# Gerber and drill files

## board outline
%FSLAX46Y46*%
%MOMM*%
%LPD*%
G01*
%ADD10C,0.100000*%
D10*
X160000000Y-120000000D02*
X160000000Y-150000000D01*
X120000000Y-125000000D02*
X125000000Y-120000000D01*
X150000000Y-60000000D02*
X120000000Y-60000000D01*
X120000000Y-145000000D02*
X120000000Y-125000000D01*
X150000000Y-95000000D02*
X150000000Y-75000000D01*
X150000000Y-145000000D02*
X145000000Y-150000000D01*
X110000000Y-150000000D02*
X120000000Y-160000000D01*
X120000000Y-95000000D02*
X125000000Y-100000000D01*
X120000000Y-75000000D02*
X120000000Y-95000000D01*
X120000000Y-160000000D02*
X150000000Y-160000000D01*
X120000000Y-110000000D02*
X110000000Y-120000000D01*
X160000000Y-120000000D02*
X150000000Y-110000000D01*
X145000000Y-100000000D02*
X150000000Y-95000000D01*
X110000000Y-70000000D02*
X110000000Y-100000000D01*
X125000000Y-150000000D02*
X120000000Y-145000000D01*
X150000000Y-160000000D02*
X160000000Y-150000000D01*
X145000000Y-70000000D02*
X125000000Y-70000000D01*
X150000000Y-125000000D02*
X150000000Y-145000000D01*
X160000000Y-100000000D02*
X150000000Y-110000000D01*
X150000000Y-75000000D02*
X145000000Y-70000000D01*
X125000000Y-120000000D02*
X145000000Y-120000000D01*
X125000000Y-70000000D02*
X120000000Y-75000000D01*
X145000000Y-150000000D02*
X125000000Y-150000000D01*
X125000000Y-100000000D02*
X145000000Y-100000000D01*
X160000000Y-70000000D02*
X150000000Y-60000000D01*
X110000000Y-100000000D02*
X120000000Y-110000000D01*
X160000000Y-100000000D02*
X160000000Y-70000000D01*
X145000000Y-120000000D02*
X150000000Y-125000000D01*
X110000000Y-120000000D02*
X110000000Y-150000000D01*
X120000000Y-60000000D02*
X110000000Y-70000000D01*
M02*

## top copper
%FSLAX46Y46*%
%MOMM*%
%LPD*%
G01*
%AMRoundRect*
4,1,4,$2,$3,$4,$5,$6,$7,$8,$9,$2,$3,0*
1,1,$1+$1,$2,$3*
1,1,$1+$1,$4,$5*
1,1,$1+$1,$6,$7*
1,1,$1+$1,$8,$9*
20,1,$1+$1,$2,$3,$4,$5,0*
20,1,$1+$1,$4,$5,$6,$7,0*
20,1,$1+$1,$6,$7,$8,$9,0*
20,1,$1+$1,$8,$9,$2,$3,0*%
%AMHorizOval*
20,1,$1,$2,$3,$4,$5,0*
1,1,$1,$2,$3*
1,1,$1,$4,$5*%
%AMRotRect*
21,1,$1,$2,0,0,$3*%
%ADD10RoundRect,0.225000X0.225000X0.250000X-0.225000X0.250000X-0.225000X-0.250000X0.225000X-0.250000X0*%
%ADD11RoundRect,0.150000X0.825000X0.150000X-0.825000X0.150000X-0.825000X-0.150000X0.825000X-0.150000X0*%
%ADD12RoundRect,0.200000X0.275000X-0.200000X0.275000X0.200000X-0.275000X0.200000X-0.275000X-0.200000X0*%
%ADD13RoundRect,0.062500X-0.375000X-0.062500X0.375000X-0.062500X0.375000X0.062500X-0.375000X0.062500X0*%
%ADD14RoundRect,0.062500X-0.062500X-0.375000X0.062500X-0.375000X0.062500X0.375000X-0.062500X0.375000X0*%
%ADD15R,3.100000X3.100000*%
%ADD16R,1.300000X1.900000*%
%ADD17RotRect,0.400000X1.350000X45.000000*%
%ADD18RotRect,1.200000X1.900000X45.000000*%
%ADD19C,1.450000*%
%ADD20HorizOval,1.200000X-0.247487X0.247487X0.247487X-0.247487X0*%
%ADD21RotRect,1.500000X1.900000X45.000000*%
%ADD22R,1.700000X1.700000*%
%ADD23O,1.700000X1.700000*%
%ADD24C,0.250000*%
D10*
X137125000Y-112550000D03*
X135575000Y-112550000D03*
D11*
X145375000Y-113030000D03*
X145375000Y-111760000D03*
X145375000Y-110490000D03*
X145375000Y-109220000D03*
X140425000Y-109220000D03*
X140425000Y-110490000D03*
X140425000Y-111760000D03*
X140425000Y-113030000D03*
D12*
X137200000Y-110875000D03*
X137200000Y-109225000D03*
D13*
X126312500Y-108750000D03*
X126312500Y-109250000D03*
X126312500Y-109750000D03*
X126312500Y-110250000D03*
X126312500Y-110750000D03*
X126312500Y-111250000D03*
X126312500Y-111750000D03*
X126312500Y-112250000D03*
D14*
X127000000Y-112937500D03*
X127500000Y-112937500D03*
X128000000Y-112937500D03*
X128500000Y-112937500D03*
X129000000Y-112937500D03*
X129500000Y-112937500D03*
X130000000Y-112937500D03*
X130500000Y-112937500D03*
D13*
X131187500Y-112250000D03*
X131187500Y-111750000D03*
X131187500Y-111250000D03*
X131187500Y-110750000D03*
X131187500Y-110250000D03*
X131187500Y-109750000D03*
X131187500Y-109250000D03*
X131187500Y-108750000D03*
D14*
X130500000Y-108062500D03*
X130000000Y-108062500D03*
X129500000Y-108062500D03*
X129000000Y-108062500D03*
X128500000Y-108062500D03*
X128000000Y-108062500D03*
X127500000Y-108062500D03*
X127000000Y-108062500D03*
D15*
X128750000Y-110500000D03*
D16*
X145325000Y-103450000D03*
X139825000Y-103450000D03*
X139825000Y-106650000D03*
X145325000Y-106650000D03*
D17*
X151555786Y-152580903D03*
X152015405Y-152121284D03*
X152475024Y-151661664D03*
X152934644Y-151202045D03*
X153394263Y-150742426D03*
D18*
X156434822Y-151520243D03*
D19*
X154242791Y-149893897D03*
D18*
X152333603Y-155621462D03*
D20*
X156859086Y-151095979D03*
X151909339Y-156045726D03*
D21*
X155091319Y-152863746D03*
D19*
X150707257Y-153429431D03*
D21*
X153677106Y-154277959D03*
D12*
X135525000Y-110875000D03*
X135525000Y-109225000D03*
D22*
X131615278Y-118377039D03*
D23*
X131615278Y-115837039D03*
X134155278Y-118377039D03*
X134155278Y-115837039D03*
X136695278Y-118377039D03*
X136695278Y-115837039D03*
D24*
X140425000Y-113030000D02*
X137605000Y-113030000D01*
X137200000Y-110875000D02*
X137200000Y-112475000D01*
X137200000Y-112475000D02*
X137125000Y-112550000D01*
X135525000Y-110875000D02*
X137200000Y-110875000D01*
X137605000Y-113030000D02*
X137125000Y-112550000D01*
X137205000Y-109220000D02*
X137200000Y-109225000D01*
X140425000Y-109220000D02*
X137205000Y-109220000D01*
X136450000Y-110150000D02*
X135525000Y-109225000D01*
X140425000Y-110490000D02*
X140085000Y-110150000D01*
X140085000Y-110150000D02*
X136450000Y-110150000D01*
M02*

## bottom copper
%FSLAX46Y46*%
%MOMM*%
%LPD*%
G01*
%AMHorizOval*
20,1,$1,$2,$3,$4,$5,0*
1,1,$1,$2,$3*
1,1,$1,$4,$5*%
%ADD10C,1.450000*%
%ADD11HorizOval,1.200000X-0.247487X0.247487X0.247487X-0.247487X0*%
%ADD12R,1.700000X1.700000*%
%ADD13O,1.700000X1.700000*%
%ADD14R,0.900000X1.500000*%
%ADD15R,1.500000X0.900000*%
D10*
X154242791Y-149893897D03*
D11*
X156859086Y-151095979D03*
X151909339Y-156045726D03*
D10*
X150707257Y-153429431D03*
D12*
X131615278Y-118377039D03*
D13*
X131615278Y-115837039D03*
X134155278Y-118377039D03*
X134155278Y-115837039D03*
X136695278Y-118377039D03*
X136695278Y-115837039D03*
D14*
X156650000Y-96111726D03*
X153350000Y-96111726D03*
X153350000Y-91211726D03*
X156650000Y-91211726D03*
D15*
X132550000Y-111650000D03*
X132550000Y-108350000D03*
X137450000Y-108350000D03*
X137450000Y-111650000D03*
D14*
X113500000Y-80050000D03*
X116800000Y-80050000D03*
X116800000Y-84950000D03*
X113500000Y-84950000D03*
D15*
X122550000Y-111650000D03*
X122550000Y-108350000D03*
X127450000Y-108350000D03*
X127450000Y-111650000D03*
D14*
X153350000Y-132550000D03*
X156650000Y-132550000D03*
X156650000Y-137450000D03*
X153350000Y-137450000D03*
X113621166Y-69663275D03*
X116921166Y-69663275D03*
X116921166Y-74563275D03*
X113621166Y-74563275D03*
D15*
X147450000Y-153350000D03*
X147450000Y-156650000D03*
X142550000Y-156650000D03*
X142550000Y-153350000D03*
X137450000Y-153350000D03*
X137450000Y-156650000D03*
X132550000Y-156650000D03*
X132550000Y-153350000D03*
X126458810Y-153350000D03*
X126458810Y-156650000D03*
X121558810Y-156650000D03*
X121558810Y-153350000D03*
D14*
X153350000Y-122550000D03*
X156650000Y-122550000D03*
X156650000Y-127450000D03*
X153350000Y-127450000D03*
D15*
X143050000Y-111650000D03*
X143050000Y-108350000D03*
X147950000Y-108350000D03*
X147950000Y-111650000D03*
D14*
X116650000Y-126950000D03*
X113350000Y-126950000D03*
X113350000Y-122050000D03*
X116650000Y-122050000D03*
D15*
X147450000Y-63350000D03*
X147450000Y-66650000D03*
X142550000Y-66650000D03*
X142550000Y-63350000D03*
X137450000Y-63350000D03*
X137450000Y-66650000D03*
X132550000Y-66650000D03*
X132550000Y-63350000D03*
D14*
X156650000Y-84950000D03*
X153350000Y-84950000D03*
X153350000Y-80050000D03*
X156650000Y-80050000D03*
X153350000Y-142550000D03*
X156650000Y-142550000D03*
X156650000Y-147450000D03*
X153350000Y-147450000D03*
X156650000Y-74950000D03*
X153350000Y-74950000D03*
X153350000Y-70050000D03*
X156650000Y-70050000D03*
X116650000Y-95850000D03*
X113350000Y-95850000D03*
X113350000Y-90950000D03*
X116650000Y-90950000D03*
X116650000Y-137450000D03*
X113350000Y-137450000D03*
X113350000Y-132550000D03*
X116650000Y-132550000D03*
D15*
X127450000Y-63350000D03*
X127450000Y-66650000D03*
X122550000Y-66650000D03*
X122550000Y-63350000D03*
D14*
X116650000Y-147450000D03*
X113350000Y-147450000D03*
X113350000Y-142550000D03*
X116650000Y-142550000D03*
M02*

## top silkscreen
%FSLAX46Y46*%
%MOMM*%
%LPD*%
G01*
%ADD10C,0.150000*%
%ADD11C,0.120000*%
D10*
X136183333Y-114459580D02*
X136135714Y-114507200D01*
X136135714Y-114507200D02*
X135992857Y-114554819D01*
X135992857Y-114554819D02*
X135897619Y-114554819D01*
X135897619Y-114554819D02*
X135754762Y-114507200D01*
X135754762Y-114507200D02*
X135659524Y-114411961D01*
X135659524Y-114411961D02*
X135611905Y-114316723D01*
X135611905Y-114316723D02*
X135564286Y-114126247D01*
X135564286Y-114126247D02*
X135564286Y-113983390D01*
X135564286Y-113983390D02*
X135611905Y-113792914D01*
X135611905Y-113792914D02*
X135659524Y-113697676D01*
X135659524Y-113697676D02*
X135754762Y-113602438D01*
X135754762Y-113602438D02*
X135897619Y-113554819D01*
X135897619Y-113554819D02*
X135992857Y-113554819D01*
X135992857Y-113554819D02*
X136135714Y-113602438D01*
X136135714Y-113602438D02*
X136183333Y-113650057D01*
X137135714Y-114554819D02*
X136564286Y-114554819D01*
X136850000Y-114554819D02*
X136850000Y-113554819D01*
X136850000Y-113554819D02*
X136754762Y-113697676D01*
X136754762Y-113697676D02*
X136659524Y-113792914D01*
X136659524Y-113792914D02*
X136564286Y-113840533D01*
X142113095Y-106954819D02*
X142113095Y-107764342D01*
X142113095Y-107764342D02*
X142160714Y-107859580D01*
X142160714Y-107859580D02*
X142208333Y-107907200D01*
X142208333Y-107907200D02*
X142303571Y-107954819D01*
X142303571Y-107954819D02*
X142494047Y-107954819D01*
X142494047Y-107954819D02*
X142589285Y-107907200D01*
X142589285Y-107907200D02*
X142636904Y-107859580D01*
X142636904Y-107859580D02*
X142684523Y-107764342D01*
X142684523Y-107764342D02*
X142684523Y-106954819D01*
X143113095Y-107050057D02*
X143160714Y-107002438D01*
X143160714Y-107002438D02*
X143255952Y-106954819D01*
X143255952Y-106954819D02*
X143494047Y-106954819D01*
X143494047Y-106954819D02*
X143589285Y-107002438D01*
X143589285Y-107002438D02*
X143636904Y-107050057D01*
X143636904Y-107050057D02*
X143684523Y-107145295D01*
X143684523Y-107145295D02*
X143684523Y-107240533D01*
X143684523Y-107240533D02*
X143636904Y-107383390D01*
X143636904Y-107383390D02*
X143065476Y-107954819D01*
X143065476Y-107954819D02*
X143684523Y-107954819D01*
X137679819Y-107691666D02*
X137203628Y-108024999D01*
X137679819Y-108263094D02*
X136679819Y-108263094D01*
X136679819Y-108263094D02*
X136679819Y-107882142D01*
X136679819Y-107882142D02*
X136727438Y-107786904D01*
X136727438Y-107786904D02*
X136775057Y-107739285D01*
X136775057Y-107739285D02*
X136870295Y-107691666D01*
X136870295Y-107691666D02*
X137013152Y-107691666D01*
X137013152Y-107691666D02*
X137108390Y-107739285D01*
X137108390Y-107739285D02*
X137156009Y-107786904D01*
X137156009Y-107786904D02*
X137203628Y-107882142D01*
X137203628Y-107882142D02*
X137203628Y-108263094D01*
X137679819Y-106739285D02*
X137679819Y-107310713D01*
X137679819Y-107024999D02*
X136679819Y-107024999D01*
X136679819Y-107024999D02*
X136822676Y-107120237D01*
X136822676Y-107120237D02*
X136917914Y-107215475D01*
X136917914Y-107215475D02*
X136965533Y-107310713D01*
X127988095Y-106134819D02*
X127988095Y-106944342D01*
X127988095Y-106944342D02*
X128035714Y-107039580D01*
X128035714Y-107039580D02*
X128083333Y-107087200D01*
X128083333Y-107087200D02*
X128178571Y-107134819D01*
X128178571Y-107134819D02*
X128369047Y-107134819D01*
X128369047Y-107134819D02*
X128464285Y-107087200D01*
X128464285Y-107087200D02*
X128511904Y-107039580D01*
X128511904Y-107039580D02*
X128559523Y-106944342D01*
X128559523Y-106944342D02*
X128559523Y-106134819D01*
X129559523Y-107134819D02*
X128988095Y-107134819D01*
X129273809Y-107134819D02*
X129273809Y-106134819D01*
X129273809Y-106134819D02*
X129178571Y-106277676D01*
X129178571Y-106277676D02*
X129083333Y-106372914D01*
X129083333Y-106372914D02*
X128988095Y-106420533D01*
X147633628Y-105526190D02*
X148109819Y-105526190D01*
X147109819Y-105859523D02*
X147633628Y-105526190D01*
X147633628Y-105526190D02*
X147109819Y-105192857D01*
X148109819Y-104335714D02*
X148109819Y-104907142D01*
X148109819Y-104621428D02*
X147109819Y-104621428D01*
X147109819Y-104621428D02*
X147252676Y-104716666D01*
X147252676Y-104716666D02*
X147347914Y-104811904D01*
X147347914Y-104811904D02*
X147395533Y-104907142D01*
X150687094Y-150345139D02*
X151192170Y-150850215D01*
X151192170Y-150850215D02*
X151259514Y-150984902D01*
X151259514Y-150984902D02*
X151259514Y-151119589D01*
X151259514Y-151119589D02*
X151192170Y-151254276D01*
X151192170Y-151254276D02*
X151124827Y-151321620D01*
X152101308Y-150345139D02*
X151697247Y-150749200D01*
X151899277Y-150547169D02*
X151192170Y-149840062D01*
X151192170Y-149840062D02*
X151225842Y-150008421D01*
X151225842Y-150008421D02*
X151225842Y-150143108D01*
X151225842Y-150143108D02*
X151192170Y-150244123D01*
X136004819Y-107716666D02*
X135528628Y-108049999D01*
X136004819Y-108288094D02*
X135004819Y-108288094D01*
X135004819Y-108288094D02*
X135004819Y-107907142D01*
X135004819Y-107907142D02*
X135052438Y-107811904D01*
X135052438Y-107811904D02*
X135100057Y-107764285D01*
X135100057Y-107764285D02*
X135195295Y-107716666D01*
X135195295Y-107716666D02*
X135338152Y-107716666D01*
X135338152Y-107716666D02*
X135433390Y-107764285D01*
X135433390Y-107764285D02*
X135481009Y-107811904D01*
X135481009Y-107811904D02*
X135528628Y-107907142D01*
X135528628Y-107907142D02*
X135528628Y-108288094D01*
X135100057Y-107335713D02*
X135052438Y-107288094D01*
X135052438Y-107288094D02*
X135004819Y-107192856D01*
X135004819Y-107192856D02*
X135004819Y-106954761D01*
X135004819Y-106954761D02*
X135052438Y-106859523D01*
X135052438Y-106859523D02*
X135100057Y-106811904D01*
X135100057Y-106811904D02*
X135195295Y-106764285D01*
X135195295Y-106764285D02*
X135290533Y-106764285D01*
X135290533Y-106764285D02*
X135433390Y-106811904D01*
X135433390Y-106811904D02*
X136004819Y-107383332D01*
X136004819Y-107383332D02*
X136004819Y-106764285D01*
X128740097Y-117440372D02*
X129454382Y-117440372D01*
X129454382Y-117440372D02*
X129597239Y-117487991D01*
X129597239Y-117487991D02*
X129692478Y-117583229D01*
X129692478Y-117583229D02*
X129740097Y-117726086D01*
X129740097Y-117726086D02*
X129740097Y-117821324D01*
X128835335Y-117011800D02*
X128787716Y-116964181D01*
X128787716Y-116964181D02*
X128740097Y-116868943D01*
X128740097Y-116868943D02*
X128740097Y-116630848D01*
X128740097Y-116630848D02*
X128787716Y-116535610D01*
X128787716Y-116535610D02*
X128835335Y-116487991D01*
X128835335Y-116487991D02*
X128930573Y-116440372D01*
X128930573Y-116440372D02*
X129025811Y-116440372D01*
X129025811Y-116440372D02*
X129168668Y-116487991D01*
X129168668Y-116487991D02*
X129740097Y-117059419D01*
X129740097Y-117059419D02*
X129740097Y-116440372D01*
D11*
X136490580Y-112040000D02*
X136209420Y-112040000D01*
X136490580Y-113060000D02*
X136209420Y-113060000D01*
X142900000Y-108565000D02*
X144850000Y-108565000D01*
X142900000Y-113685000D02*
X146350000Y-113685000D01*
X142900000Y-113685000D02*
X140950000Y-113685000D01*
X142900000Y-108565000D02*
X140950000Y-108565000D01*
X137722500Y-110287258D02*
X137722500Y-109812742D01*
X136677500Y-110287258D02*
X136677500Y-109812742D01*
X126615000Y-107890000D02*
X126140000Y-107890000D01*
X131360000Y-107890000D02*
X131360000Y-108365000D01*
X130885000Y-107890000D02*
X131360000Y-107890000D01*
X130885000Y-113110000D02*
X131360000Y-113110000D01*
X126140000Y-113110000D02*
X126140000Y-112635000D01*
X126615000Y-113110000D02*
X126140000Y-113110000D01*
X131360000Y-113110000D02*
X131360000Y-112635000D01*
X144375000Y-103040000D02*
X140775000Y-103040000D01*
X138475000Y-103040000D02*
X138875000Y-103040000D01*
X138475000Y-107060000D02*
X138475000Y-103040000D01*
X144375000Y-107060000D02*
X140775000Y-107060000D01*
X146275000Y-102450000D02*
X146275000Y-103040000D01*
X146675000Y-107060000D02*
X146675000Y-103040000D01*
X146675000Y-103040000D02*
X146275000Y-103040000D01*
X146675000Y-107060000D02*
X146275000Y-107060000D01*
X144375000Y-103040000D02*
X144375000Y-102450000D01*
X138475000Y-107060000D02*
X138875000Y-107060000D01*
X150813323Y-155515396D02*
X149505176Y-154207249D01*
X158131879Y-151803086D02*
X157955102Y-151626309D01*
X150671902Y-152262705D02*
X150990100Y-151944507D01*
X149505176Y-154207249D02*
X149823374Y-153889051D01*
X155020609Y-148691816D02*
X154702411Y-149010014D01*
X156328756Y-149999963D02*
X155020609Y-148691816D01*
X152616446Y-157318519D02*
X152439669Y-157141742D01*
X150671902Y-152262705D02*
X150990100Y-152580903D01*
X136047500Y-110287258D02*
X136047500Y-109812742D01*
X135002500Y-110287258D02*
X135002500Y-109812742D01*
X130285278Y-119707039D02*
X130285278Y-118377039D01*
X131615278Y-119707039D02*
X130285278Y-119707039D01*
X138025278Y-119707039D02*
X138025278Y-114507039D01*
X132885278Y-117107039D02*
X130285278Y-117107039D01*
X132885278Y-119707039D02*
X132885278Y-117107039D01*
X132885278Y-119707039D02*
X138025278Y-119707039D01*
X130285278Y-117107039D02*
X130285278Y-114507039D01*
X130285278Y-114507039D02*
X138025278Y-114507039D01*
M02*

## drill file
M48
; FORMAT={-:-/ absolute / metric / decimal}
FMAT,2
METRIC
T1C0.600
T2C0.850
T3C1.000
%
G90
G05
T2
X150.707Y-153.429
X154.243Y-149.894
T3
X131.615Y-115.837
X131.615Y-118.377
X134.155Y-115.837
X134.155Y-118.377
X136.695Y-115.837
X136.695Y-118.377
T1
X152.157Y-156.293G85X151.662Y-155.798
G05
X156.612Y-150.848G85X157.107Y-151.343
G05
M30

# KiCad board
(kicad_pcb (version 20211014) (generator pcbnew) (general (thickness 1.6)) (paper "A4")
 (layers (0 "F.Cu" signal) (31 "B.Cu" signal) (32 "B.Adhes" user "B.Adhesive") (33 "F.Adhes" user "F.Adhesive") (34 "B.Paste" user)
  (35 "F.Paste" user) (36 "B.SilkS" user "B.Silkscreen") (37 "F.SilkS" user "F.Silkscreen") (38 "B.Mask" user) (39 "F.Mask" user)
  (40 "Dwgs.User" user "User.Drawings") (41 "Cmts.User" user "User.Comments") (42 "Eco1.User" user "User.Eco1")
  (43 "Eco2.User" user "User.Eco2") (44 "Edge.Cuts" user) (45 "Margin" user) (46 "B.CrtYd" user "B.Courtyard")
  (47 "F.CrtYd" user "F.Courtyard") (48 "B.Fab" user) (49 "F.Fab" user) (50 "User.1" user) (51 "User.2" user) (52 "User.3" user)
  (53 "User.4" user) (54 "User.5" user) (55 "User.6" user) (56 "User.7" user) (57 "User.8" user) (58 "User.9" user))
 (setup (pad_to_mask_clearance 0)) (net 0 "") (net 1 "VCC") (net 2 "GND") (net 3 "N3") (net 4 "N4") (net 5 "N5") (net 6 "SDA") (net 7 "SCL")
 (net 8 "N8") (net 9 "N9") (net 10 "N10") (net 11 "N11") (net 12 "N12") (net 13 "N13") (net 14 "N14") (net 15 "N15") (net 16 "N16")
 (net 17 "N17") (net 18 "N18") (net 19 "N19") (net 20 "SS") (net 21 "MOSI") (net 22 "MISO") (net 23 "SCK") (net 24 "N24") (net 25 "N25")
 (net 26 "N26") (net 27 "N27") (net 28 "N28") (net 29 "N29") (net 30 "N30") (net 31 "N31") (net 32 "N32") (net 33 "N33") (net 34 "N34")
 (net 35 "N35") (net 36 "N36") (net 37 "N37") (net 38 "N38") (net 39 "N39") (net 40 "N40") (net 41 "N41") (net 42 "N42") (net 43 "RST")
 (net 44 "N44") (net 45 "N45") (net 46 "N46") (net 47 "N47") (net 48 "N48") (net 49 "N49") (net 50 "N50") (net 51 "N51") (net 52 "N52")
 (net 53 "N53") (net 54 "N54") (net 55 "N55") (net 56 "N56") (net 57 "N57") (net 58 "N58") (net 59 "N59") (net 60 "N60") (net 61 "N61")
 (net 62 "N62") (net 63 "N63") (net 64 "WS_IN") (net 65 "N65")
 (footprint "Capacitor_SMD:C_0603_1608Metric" (layer "F.Cu") (at 136.35 112.55 180)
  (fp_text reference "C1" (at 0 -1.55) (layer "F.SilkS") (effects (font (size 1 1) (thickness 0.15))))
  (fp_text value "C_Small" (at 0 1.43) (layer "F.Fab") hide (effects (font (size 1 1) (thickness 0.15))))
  (fp_line (start -0.14058 0.51) (end 0.14058 0.51) (layer "F.SilkS") (width 0.12))
  (fp_line (start -0.14058 -0.51) (end 0.14058 -0.51) (layer "F.SilkS") (width 0.12))
  (pad "1" smd roundrect (at -0.775 0 180) (size 0.9 0.95) (layers "F.Cu" "F.Paste" "F.Mask") (roundrect_rratio 0.25) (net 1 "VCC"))
  (pad "2" smd roundrect (at 0.775 0 180) (size 0.9 0.95) (layers "F.Cu" "F.Paste" "F.Mask") (roundrect_rratio 0.25) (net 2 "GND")))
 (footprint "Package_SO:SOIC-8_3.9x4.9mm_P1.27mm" (layer "F.Cu") (at 142.9 111.125 180)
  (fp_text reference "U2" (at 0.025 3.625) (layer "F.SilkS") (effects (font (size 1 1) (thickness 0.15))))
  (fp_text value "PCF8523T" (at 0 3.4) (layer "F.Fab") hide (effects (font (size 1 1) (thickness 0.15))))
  (fp_line (start 0 2.56) (end -1.95 2.56) (layer "F.SilkS") (width 0.12))
  (fp_line (start 0 -2.56) (end -3.45 -2.56) (layer "F.SilkS") (width 0.12))
  (fp_line (start 0 -2.56) (end 1.95 -2.56) (layer "F.SilkS") (width 0.12))
  (fp_line (start 0 2.56) (end 1.95 2.56) (layer "F.SilkS") (width 0.12))
  (pad "1" smd roundrect (at -2.475 -1.905 180) (size 1.95 0.6) (layers "F.Cu" "F.Paste" "F.Mask") (roundrect_rratio 0.25) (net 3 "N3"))
  (pad "2" smd roundrect (at -2.475 -0.635 180) (size 1.95 0.6) (layers "F.Cu" "F.Paste" "F.Mask") (roundrect_rratio 0.25) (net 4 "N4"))
  (pad "3" smd roundrect (at -2.475 0.635 180) (size 1.95 0.6) (layers "F.Cu" "F.Paste" "F.Mask") (roundrect_rratio 0.25) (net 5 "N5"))
  (pad "4" smd roundrect (at -2.475 1.905 180) (size 1.95 0.6) (layers "F.Cu" "F.Paste" "F.Mask") (roundrect_rratio 0.25) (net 2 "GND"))
  (pad "5" smd roundrect (at 2.475 1.905 180) (size 1.95 0.6) (layers "F.Cu" "F.Paste" "F.Mask") (roundrect_rratio 0.25) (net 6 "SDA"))
  (pad "6" smd roundrect (at 2.475 0.635 180) (size 1.95 0.6) (layers "F.Cu" "F.Paste" "F.Mask") (roundrect_rratio 0.25) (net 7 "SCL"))
  (pad "7" smd roundrect (at 2.475 -0.635 180) (size 1.95 0.6) (layers "F.Cu" "F.Paste" "F.Mask") (roundrect_rratio 0.25) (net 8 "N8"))
  (pad "8" smd roundrect (at 2.475 -1.905 180) (size 1.95 0.6) (layers "F.Cu" "F.Paste" "F.Mask") (roundrect_rratio 0.25) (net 1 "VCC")))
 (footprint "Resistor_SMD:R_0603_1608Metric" (layer "F.Cu") (at 137.2 110.05 90)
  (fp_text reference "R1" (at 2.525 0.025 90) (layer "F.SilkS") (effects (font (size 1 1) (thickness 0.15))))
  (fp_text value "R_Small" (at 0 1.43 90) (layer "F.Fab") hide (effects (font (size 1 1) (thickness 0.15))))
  (fp_line (start -0.237258 0.5225) (end 0.237258 0.5225) (layer "F.SilkS") (width 0.12))
  (fp_line (start -0.237258 -0.5225) (end 0.237258 -0.5225) (layer "F.SilkS") (width 0.12))
  (pad "1" smd roundrect (at -0.825 0 90) (size 0.8 0.95) (layers "F.Cu" "F.Paste" "F.Mask") (roundrect_rratio 0.25) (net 1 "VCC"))
  (pad "2" smd roundrect (at 0.825 0 90) (size 0.8 0.95) (layers "F.Cu" "F.Paste" "F.Mask") (roundrect_rratio 0.25) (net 6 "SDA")))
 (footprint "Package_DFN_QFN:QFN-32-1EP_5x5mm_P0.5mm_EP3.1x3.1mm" (layer "F.Cu") (at 128.75 110.5)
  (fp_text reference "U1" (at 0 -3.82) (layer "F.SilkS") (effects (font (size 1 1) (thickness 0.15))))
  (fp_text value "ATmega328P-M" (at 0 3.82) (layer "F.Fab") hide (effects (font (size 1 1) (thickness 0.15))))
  (fp_line (start -2.135 -2.61) (end -2.61 -2.61) (layer "F.SilkS") (width 0.12))
  (fp_line (start 2.61 -2.61) (end 2.61 -2.135) (layer "F.SilkS") (width 0.12))
  (fp_line (start 2.135 -2.61) (end 2.61 -2.61) (layer "F.SilkS") (width 0.12))
  (fp_line (start 2.135 2.61) (end 2.61 2.61) (layer "F.SilkS") (width 0.12))
  (fp_line (start -2.61 2.61) (end -2.61 2.135) (layer "F.SilkS") (width 0.12))
  (fp_line (start -2.135 2.61) (end -2.61 2.61) (layer "F.SilkS") (width 0.12))
  (fp_line (start 2.61 2.61) (end 2.61 2.135) (layer "F.SilkS") (width 0.12))
  (pad "" smd roundrect (at 1.03 -1.03) (size 0.83 0.83) (layers "F.Paste") (roundrect_rratio 0.25))
  (pad "" smd roundrect (at -1.03 -1.03) (size 0.83 0.83) (layers "F.Paste") (roundrect_rratio 0.25))
  (pad "" smd roundrect (at 1.03 0) (size 0.83 0.83) (layers "F.Paste") (roundrect_rratio 0.25))
  (pad "" smd roundrect (at -1.03 1.03) (size 0.83 0.83) (layers "F.Paste") (roundrect_rratio 0.25))
  (pad "" smd roundrect (at -1.03 0) (size 0.83 0.83) (layers "F.Paste") (roundrect_rratio 0.25))
  (pad "" smd roundrect (at 0 1.03) (size 0.83 0.83) (layers "F.Paste") (roundrect_rratio 0.25))
  (pad "" smd roundrect (at 0 0) (size 0.83 0.83) (layers "F.Paste") (roundrect_rratio 0.25))
  (pad "" smd roundrect (at 0 -1.03) (size 0.83 0.83) (layers "F.Paste") (roundrect_rratio 0.25))
  (pad "" smd roundrect (at 1.03 1.03) (size 0.83 0.83) (layers "F.Paste") (roundrect_rratio 0.25))
  (pad "1" smd roundrect (at -2.4375 -1.75) (size 0.875 0.25) (layers "F.Cu" "F.Paste" "F.Mask") (roundrect_rratio 0.25) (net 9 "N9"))
  (pad "2" smd roundrect (at -2.4375 -1.25) (size 0.875 0.25) (layers "F.Cu" "F.Paste" "F.Mask") (roundrect_rratio 0.25) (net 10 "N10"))
  (pad "3" smd roundrect (at -2.4375 -0.75) (size 0.875 0.25) (layers "F.Cu" "F.Paste" "F.Mask") (roundrect_rratio 0.25) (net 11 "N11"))
  (pad "4" smd roundrect (at -2.4375 -0.25) (size 0.875 0.25) (layers "F.Cu" "F.Paste" "F.Mask") (roundrect_rratio 0.25) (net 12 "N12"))
  (pad "5" smd roundrect (at -2.4375 0.25) (size 0.875 0.25) (layers "F.Cu" "F.Paste" "F.Mask") (roundrect_rratio 0.25) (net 11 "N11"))
  (pad "6" smd roundrect (at -2.4375 0.75) (size 0.875 0.25) (layers "F.Cu" "F.Paste" "F.Mask") (roundrect_rratio 0.25) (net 12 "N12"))
  (pad "7" smd roundrect (at -2.4375 1.25) (size 0.875 0.25) (layers "F.Cu" "F.Paste" "F.Mask") (roundrect_rratio 0.25) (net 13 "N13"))
  (pad "8" smd roundrect (at -2.4375 1.75) (size 0.875 0.25) (layers "F.Cu" "F.Paste" "F.Mask") (roundrect_rratio 0.25) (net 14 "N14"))
  (pad "9" smd roundrect (at -1.75 2.4375) (size 0.25 0.875) (layers "F.Cu" "F.Paste" "F.Mask") (roundrect_rratio 0.25) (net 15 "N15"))
  (pad "10" smd roundrect (at -1.25 2.4375) (size 0.25 0.875) (layers "F.Cu" "F.Paste" "F.Mask") (roundrect_rratio 0.25) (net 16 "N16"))
  (pad "11" smd roundrect (at -0.75 2.4375) (size 0.25 0.875) (layers "F.Cu" "F.Paste" "F.Mask") (roundrect_rratio 0.25) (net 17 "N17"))
  (pad "12" smd roundrect (at -0.25 2.4375) (size 0.25 0.875) (layers "F.Cu" "F.Paste" "F.Mask") (roundrect_rratio 0.25) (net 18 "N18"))
  (pad "13" smd roundrect (at 0.25 2.4375) (size 0.25 0.875) (layers "F.Cu" "F.Paste" "F.Mask") (roundrect_rratio 0.25) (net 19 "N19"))
  (pad "14" smd roundrect (at 0.75 2.4375) (size 0.25 0.875) (layers "F.Cu" "F.Paste" "F.Mask") (roundrect_rratio 0.25) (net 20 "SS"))
  (pad "15" smd roundrect (at 1.25 2.4375) (size 0.25 0.875) (layers "F.Cu" "F.Paste" "F.Mask") (roundrect_rratio 0.25) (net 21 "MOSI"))
  (pad "16" smd roundrect (at 1.75 2.4375) (size 0.25 0.875) (layers "F.Cu" "F.Paste" "F.Mask") (roundrect_rratio 0.25) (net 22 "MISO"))
  (pad "17" smd roundrect (at 2.4375 1.75) (size 0.875 0.25) (layers "F.Cu" "F.Paste" "F.Mask") (roundrect_rratio 0.25) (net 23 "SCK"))
  (pad "18" smd roundrect (at 2.4375 1.25) (size 0.875 0.25) (layers "F.Cu" "F.Paste" "F.Mask") (roundrect_rratio 0.25) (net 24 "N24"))
  (pad "19" smd roundrect (at 2.4375 0.75) (size 0.875 0.25) (layers "F.Cu" "F.Paste" "F.Mask") (roundrect_rratio 0.25) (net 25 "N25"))
  (pad "20" smd roundrect (at 2.4375 0.25) (size 0.875 0.25) (layers "F.Cu" "F.Paste" "F.Mask") (roundrect_rratio 0.25) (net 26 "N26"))
  (pad "21" smd roundrect (at 2.4375 -0.25) (size 0.875 0.25) (layers "F.Cu" "F.Paste" "F.Mask") (roundrect_rratio 0.25) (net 11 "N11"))
  (pad "22" smd roundrect (at 2.4375 -0.75) (size 0.875 0.25) (layers "F.Cu" "F.Paste" "F.Mask") (roundrect_rratio 0.25) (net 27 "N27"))
  (pad "23" smd roundrect (at 2.4375 -1.25) (size 0.875 0.25) (layers "F.Cu" "F.Paste" "F.Mask") (roundrect_rratio 0.25) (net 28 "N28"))
  (pad "24" smd roundrect (at 2.4375 -1.75) (size 0.875 0.25) (layers "F.Cu" "F.Paste" "F.Mask") (roundrect_rratio 0.25) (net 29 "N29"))
  (pad "25" smd roundrect (at 1.75 -2.4375) (size 0.25 0.875) (layers "F.Cu" "F.Paste" "F.Mask") (roundrect_rratio 0.25) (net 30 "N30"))
  (pad "26" smd roundrect (at 1.25 -2.4375) (size 0.25 0.875) (layers "F.Cu" "F.Paste" "F.Mask") (roundrect_rratio 0.25) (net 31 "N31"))
  (pad "27" smd roundrect (at 0.75 -2.4375) (size 0.25 0.875) (layers "F.Cu" "F.Paste" "F.Mask") (roundrect_rratio 0.25) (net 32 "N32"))
  (pad "28" smd roundrect (at 0.25 -2.4375) (size 0.25 0.875) (layers "F.Cu" "F.Paste" "F.Mask") (roundrect_rratio 0.25) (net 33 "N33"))
  (pad "29" smd roundrect (at -0.25 -2.4375) (size 0.25 0.875) (layers "F.Cu" "F.Paste" "F.Mask") (roundrect_rratio 0.25) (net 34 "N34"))
  (pad "30" smd roundrect (at -0.75 -2.4375) (size 0.25 0.875) (layers "F.Cu" "F.Paste" "F.Mask") (roundrect_rratio 0.25) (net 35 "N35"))
  (pad "31" smd roundrect (at -1.25 -2.4375) (size 0.25 0.875) (layers "F.Cu" "F.Paste" "F.Mask") (roundrect_rratio 0.25) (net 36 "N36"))
  (pad "32" smd roundrect (at -1.75 -2.4375) (size 0.25 0.875) (layers "F.Cu" "F.Paste" "F.Mask") (roundrect_rratio 0.25) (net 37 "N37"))
  (pad "33" smd rect (at 0 0) (size 3.1 3.1) (layers "F.Cu" "F.Mask") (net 11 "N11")))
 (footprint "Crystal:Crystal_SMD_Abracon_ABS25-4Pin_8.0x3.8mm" (layer "F.Cu") (at 142.575 105.05 -90)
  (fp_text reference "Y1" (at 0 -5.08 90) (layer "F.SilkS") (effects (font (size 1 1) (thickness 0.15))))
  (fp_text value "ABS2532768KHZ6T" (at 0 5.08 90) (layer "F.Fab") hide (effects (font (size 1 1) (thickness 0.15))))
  (fp_line (start -2.01 -1.8) (end -2.01 1.8) (layer "F.SilkS") (width 0.12))
  (fp_line (start -2.01 4.1) (end -2.01 3.7) (layer "F.SilkS") (width 0.12))
  (fp_line (start 2.01 4.1) (end -2.01 4.1) (layer "F.SilkS") (width 0.12))
  (fp_line (start 2.01 -1.8) (end 2.01 1.8) (layer "F.SilkS") (width 0.12))
  (fp_line (start -2.6 -3.7) (end -2.01 -3.7) (layer "F.SilkS") (width 0.12))
  (fp_line (start 2.01 -4.1) (end -2.01 -4.1) (layer "F.SilkS") (width 0.12))
  (fp_line (start -2.01 -4.1) (end -2.01 -3.7) (layer "F.SilkS") (width 0.12))
  (fp_line (start 2.01 -4.1) (end 2.01 -3.7) (layer "F.SilkS") (width 0.12))
  (fp_line (start -2.01 -1.8) (end -2.6 -1.8) (layer "F.SilkS") (width 0.12))
  (fp_line (start 2.01 4.1) (end 2.01 3.7) (layer "F.SilkS") (width 0.12))
  (pad "1" smd rect (at -1.6 -2.75 180) (size 1.3 1.9) (layers "F.Cu" "F.Paste" "F.Mask") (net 3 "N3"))
  (pad "2" smd rect (at -1.6 2.75 180) (size 1.3 1.9) (layers "F.Cu" "F.Paste" "F.Mask") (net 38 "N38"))
  (pad "3" smd rect (at 1.6 2.75 180) (size 1.3 1.9) (layers "F.Cu" "F.Paste" "F.Mask") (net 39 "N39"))
  (pad "4" smd rect (at 1.6 -2.75 180) (size 1.3 1.9) (layers "F.Cu" "F.Paste" "F.Mask") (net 4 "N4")))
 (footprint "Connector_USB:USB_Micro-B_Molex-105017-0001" (layer "F.Cu") (at 153.509168 152.695808 45)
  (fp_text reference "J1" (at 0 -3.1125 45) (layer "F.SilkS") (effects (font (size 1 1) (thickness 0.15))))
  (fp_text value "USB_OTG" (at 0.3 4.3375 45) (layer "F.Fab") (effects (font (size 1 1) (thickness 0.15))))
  (fp_line (start -3.9 0.0875) (end -3.9 -1.7625) (layer "F.SilkS") (width 0.12))
  (fp_line (start 3.9 2.6375) (end 3.9 2.3875) (layer "F.SilkS") (width 0.12))
  (fp_line (start -1.7 -2.3125) (end -1.25 -2.3125) (layer "F.SilkS") (width 0.12))
  (fp_line (start -3.9 -1.7625) (end -3.45 -1.7625) (layer "F.SilkS") (width 0.12))
  (fp_line (start 3.9 -1.7625) (end 3.45 -1.7625) (layer "F.SilkS") (width 0.12))
  (fp_line (start 3.9 0.0875) (end 3.9 -1.7625) (layer "F.SilkS") (width 0.12))
  (fp_line (start -3.9 2.6375) (end -3.9 2.3875) (layer "F.SilkS") (width 0.12))
  (fp_line (start -1.7 -2.3125) (end -1.7 -1.8625) (layer "F.SilkS") (width 0.12))
  (pad "1" smd rect (at -1.3 -1.4625 45) (size 0.4 1.35) (layers "F.Cu" "F.Paste" "F.Mask") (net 1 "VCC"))
  (pad "2" smd rect (at -0.65 -1.4625 45) (size 0.4 1.35) (layers "F.Cu" "F.Paste" "F.Mask") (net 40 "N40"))
  (pad "3" smd rect (at 0 -1.4625 45) (size 0.4 1.35) (layers "F.Cu" "F.Paste" "F.Mask") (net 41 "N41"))
  (pad "4" smd rect (at 0.65 -1.4625 45) (size 0.4 1.35) (layers "F.Cu" "F.Paste" "F.Mask") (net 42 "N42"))
  (pad "5" smd rect (at 1.3 -1.4625 45) (size 0.4 1.35) (layers "F.Cu" "F.Paste" "F.Mask") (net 2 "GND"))
  (pad "6" smd rect (at 2.9 1.2375 45) (size 1.2 1.9) (layers "F.Cu" "F.Mask") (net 2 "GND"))
  (pad "6" thru_hole circle (at 2.5 -1.4625 45) (size 1.45 1.45) (drill 0.85) (layers *.Cu *.Mask) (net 2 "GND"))
  (pad "6" smd rect (at -2.9 1.2375 45) (size 1.2 1.9) (layers "F.Cu" "F.Mask") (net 2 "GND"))
  (pad "6" thru_hole oval (at 3.5 1.2375 45) (size 1.2 1.9) (drill oval 0.6 1.3) (layers *.Cu *.Mask) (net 2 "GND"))
  (pad "6" thru_hole oval (at -3.5 1.2375 225) (size 1.2 1.9) (drill oval 0.6 1.3) (layers *.Cu *.Mask) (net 2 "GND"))
  (pad "6" smd rect (at 1 1.2375 45) (size 1.5 1.9) (layers "F.Cu" "F.Paste" "F.Mask") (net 2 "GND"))
  (pad "6" thru_hole circle (at -2.5 -1.4625 45) (size 1.45 1.45) (drill 0.85) (layers *.Cu *.Mask) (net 2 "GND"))
  (pad "6" smd rect (at -1 1.2375 45) (size 1.5 1.9) (layers "F.Cu" "F.Paste" "F.Mask") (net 2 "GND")))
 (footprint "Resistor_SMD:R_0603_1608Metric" (layer "F.Cu") (at 135.525 110.05 90)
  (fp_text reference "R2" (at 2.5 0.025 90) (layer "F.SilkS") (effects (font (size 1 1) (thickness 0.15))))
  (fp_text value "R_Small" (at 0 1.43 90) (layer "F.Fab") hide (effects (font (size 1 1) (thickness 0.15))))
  (fp_line (start -0.237258 0.5225) (end 0.237258 0.5225) (layer "F.SilkS") (width 0.12))
  (fp_line (start -0.237258 -0.5225) (end 0.237258 -0.5225) (layer "F.SilkS") (width 0.12))
  (pad "1" smd roundrect (at -0.825 0 90) (size 0.8 0.95) (layers "F.Cu" "F.Paste" "F.Mask") (roundrect_rratio 0.25) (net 1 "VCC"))
  (pad "2" smd roundrect (at 0.825 0 90) (size 0.8 0.95) (layers "F.Cu" "F.Paste" "F.Mask") (roundrect_rratio 0.25) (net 7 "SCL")))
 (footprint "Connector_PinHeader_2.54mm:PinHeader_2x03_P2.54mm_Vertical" (layer "F.Cu") (at 131.615278 118.377039 90)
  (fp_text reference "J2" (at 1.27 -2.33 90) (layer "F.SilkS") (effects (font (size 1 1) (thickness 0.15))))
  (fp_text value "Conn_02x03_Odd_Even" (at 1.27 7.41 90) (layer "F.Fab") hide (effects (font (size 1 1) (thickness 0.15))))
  (fp_line (start -1.33 -1.33) (end 0 -1.33) (layer "F.SilkS") (width 0.12))
  (fp_line (start -1.33 0) (end -1.33 -1.33) (layer "F.SilkS") (width 0.12))
  (fp_line (start -1.33 6.41) (end 3.87 6.41) (layer "F.SilkS") (width 0.12))
  (fp_line (start 1.27 1.27) (end 1.27 -1.33) (layer "F.SilkS") (width 0.12))
  (fp_line (start -1.33 1.27) (end 1.27 1.27) (layer "F.SilkS") (width 0.12))
  (fp_line (start -1.33 1.27) (end -1.33 6.41) (layer "F.SilkS") (width 0.12))
  (fp_line (start 1.27 -1.33) (end 3.87 -1.33) (layer "F.SilkS") (width 0.12))
  (fp_line (start 3.87 -1.33) (end 3.87 6.41) (layer "F.SilkS") (width 0.12))
  (pad "1" thru_hole rect (at 0 0 90) (size 1.7 1.7) (drill 1) (layers *.Cu *.Mask) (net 22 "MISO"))
  (pad "2" thru_hole oval (at 2.54 0 90) (size 1.7 1.7) (drill 1) (layers *.Cu *.Mask) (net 1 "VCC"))
  (pad "3" thru_hole oval (at 0 2.54 90) (size 1.7 1.7) (drill 1) (layers *.Cu *.Mask) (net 23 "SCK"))
  (pad "4" thru_hole oval (at 2.54 2.54 90) (size 1.7 1.7) (drill 1) (layers *.Cu *.Mask) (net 21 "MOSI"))
  (pad "5" thru_hole oval (at 0 5.08 90) (size 1.7 1.7) (drill 1) (layers *.Cu *.Mask) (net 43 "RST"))
  (pad "6" thru_hole oval (at 2.54 5.08 90) (size 1.7 1.7) (drill 1) (layers *.Cu *.Mask) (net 2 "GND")))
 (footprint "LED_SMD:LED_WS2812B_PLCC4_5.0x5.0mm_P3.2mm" (layer "B.Cu") (at 155 93.661726 90)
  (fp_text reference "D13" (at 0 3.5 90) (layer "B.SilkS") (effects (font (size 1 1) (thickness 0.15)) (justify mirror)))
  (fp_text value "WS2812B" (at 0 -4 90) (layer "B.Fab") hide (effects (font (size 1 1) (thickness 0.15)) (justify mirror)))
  (pad "1" smd rect (at -2.45 1.65 90) (size 1.5 0.9) (layers "B.Cu" "B.Paste" "B.Mask") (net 1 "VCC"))
  (pad "2" smd rect (at -2.45 -1.65 90) (size 1.5 0.9) (layers "B.Cu" "B.Paste" "B.Mask") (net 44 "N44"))
  (pad "3" smd rect (at 2.45 -1.65 90) (size 1.5 0.9) (layers "B.Cu" "B.Paste" "B.Mask") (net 2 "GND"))
  (pad "4" smd rect (at 2.45 1.65 90) (size 1.5 0.9) (layers "B.Cu" "B.Paste" "B.Mask") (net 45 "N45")))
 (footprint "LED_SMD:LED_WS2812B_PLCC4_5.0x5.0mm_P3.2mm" (layer "B.Cu") (at 135 110)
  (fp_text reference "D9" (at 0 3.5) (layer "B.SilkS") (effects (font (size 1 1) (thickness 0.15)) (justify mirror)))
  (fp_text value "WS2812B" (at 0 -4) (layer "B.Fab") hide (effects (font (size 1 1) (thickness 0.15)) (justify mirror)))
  (pad "1" smd rect (at -2.45 1.65) (size 1.5 0.9) (layers "B.Cu" "B.Paste" "B.Mask") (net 1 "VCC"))
  (pad "2" smd rect (at -2.45 -1.65) (size 1.5 0.9) (layers "B.Cu" "B.Paste" "B.Mask") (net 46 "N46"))
  (pad "3" smd rect (at 2.45 -1.65) (size 1.5 0.9) (layers "B.Cu" "B.Paste" "B.Mask") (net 2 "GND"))
  (pad "4" smd rect (at 2.45 1.65) (size 1.5 0.9) (layers "B.Cu" "B.Paste" "B.Mask") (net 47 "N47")))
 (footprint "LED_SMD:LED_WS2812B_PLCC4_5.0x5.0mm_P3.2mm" (layer "B.Cu") (at 115.15 82.5 -90)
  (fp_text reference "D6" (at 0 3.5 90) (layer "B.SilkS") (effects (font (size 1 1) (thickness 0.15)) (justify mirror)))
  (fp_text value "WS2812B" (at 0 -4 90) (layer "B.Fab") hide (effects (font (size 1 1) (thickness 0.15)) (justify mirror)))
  (pad "1" smd rect (at -2.45 1.65 270) (size 1.5 0.9) (layers "B.Cu" "B.Paste" "B.Mask") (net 1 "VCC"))
  (pad "2" smd rect (at -2.45 -1.65 270) (size 1.5 0.9) (layers "B.Cu" "B.Paste" "B.Mask") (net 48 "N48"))
  (pad "3" smd rect (at 2.45 -1.65 270) (size 1.5 0.9) (layers "B.Cu" "B.Paste" "B.Mask") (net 2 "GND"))
  (pad "4" smd rect (at 2.45 1.65 270) (size 1.5 0.9) (layers "B.Cu" "B.Paste" "B.Mask") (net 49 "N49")))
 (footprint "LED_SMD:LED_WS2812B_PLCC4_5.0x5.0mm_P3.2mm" (layer "B.Cu") (at 125 110)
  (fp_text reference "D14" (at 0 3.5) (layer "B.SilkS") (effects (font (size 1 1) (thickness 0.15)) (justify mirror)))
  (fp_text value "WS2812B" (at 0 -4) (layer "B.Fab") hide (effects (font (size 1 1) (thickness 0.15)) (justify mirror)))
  (pad "1" smd rect (at -2.45 1.65) (size 1.5 0.9) (layers "B.Cu" "B.Paste" "B.Mask") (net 1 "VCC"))
  (pad "2" smd rect (at -2.45 -1.65) (size 1.5 0.9) (layers "B.Cu" "B.Paste" "B.Mask") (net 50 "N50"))
  (pad "3" smd rect (at 2.45 -1.65) (size 1.5 0.9) (layers "B.Cu" "B.Paste" "B.Mask") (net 2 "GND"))
  (pad "4" smd rect (at 2.45 1.65) (size 1.5 0.9) (layers "B.Cu" "B.Paste" "B.Mask") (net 46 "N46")))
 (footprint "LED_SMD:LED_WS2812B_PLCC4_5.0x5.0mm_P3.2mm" (layer "B.Cu") (at 155 135 -90)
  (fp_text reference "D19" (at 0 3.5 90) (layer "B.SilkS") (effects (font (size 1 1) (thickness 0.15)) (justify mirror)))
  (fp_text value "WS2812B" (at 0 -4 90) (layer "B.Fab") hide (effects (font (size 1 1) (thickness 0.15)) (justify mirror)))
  (pad "1" smd rect (at -2.45 1.65 270) (size 1.5 0.9) (layers "B.Cu" "B.Paste" "B.Mask") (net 1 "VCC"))
  (pad "2" smd rect (at -2.45 -1.65 270) (size 1.5 0.9) (layers "B.Cu" "B.Paste" "B.Mask") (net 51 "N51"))
  (pad "3" smd rect (at 2.45 -1.65 270) (size 1.5 0.9) (layers "B.Cu" "B.Paste" "B.Mask") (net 2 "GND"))
  (pad "4" smd rect (at 2.45 1.65 270) (size 1.5 0.9) (layers "B.Cu" "B.Paste" "B.Mask") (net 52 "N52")))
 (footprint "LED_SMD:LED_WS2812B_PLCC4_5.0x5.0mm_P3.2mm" (layer "B.Cu") (at 115.271166 72.113275 -90)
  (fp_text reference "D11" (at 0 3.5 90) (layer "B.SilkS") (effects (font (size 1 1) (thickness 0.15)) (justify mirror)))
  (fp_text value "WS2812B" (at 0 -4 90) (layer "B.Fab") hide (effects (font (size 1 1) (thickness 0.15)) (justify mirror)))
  (pad "1" smd rect (at -2.45 1.65 270) (size 1.5 0.9) (layers "B.Cu" "B.Paste" "B.Mask") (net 1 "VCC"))
  (pad "2" smd rect (at -2.45 -1.65 270) (size 1.5 0.9) (layers "B.Cu" "B.Paste" "B.Mask") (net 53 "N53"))
  (pad "3" smd rect (at 2.45 -1.65 270) (size 1.5 0.9) (layers "B.Cu" "B.Paste" "B.Mask") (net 2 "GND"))
  (pad "4" smd rect (at 2.45 1.65 270) (size 1.5 0.9) (layers "B.Cu" "B.Paste" "B.Mask") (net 48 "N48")))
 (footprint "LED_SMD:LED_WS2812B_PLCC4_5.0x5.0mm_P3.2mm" (layer "B.Cu") (at 145 155 180)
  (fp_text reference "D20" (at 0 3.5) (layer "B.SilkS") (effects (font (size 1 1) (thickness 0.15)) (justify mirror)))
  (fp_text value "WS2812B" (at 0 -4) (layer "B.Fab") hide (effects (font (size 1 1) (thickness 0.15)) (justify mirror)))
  (pad "1" smd rect (at -2.45 1.65 180) (size 1.5 0.9) (layers "B.Cu" "B.Paste" "B.Mask") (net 1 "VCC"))
  (pad "2" smd rect (at -2.45 -1.65 180) (size 1.5 0.9) (layers "B.Cu" "B.Paste" "B.Mask") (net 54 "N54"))
  (pad "3" smd rect (at 2.45 -1.65 180) (size 1.5 0.9) (layers "B.Cu" "B.Paste" "B.Mask") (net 2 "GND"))
  (pad "4" smd rect (at 2.45 1.65 180) (size 1.5 0.9) (layers "B.Cu" "B.Paste" "B.Mask") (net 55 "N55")))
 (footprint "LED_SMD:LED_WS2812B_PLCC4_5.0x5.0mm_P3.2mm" (layer "B.Cu") (at 135 155 180)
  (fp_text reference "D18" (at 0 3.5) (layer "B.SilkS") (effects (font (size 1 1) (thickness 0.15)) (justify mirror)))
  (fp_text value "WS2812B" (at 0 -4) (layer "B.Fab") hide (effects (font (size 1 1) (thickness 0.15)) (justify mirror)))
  (pad "1" smd rect (at -2.45 1.65 180) (size 1.5 0.9) (layers "B.Cu" "B.Paste" "B.Mask") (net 1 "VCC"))
  (pad "2" smd rect (at -2.45 -1.65 180) (size 1.5 0.9) (layers "B.Cu" "B.Paste" "B.Mask") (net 55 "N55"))
  (pad "3" smd rect (at 2.45 -1.65 180) (size 1.5 0.9) (layers "B.Cu" "B.Paste" "B.Mask") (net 2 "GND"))
  (pad "4" smd rect (at 2.45 1.65 180) (size 1.5 0.9) (layers "B.Cu" "B.Paste" "B.Mask") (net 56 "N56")))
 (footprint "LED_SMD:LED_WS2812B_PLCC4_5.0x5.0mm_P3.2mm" (layer "B.Cu") (at 124.00881 155 180)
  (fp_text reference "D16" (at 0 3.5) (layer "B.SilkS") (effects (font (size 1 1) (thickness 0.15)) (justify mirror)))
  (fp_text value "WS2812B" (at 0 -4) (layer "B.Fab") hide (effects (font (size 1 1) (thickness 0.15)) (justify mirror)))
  (pad "1" smd rect (at -2.45 1.65 180) (size 1.5 0.9) (layers "B.Cu" "B.Paste" "B.Mask") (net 1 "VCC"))
  (pad "2" smd rect (at -2.45 -1.65 180) (size 1.5 0.9) (layers "B.Cu" "B.Paste" "B.Mask") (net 56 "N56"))
  (pad "3" smd rect (at 2.45 -1.65 180) (size 1.5 0.9) (layers "B.Cu" "B.Paste" "B.Mask") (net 2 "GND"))
  (pad "4" smd rect (at 2.45 1.65 180) (size 1.5 0.9) (layers "B.Cu" "B.Paste" "B.Mask") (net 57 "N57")))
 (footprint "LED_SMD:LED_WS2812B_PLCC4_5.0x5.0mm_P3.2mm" (layer "B.Cu") (at 155 125 -90)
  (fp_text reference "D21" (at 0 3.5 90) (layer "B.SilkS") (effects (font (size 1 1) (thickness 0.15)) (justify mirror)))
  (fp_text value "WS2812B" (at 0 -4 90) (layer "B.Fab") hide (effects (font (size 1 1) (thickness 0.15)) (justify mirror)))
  (pad "1" smd rect (at -2.45 1.65 270) (size 1.5 0.9) (layers "B.Cu" "B.Paste" "B.Mask") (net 1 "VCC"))
  (pad "2" smd rect (at -2.45 -1.65 270) (size 1.5 0.9) (layers "B.Cu" "B.Paste" "B.Mask") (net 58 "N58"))
  (pad "3" smd rect (at 2.45 -1.65 270) (size 1.5 0.9) (layers "B.Cu" "B.Paste" "B.Mask") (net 2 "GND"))
  (pad "4" smd rect (at 2.45 1.65 270) (size 1.5 0.9) (layers "B.Cu" "B.Paste" "B.Mask") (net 51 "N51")))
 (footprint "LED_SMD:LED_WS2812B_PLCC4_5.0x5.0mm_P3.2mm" (layer "B.Cu") (at 145.5 110)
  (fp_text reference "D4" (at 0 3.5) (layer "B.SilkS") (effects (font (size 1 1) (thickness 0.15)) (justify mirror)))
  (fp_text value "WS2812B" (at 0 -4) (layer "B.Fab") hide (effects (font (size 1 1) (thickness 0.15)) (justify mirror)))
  (pad "1" smd rect (at -2.45 1.65) (size 1.5 0.9) (layers "B.Cu" "B.Paste" "B.Mask") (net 1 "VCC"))
  (pad "2" smd rect (at -2.45 -1.65) (size 1.5 0.9) (layers "B.Cu" "B.Paste" "B.Mask") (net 47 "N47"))
  (pad "3" smd rect (at 2.45 -1.65) (size 1.5 0.9) (layers "B.Cu" "B.Paste" "B.Mask") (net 2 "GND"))
  (pad "4" smd rect (at 2.45 1.65) (size 1.5 0.9) (layers "B.Cu" "B.Paste" "B.Mask") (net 44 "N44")))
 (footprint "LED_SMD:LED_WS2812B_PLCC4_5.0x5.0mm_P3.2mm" (layer "B.Cu") (at 115 124.5 90)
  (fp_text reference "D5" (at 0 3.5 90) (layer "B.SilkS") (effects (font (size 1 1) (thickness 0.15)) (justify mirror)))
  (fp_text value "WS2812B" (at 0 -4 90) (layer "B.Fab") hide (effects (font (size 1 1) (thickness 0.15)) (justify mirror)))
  (pad "1" smd rect (at -2.45 1.65 90) (size 1.5 0.9) (layers "B.Cu" "B.Paste" "B.Mask") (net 1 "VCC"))
  (pad "2" smd rect (at -2.45 -1.65 90) (size 1.5 0.9) (layers "B.Cu" "B.Paste" "B.Mask") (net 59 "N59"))
  (pad "3" smd rect (at 2.45 -1.65 90) (size 1.5 0.9) (layers "B.Cu" "B.Paste" "B.Mask") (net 2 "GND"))
  (pad "4" smd rect (at 2.45 1.65 90) (size 1.5 0.9) (layers "B.Cu" "B.Paste" "B.Mask") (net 50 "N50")))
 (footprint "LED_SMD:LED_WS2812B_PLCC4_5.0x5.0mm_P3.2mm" (layer "B.Cu") (at 145 65 180)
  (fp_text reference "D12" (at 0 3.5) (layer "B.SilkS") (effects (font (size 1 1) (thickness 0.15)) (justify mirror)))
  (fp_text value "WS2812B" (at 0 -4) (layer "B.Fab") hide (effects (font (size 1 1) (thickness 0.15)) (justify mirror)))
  (pad "1" smd rect (at -2.45 1.65 180) (size 1.5 0.9) (layers "B.Cu" "B.Paste" "B.Mask") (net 1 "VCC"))
  (pad "2" smd rect (at -2.45 -1.65 180) (size 1.5 0.9) (layers "B.Cu" "B.Paste" "B.Mask") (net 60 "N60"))
  (pad "3" smd rect (at 2.45 -1.65 180) (size 1.5 0.9) (layers "B.Cu" "B.Paste" "B.Mask") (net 2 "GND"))
  (pad "4" smd rect (at 2.45 1.65 180) (size 1.5 0.9) (layers "B.Cu" "B.Paste" "B.Mask") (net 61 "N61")))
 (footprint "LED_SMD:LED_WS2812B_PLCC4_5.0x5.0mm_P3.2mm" (layer "B.Cu") (at 135 65 180)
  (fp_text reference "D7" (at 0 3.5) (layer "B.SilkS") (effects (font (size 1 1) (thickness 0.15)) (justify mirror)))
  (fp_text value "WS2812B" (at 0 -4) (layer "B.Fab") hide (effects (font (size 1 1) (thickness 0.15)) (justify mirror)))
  (pad "1" smd rect (at -2.45 1.65 180) (size 1.5 0.9) (layers "B.Cu" "B.Paste" "B.Mask") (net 1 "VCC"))
  (pad "2" smd rect (at -2.45 -1.65 180) (size 1.5 0.9) (layers "B.Cu" "B.Paste" "B.Mask") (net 61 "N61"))
  (pad "3" smd rect (at 2.45 -1.65 180) (size 1.5 0.9) (layers "B.Cu" "B.Paste" "B.Mask") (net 2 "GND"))
  (pad "4" smd rect (at 2.45 1.65 180) (size 1.5 0.9) (layers "B.Cu" "B.Paste" "B.Mask") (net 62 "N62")))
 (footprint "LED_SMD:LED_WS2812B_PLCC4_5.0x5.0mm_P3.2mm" (layer "B.Cu") (at 155 82.5 90)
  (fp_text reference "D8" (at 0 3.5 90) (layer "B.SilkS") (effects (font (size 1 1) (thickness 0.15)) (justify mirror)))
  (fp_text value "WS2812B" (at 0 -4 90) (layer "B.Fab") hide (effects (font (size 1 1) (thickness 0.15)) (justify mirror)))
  (pad "1" smd rect (at -2.45 1.65 90) (size 1.5 0.9) (layers "B.Cu" "B.Paste" "B.Mask") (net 1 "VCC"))
  (pad "2" smd rect (at -2.45 -1.65 90) (size 1.5 0.9) (layers "B.Cu" "B.Paste" "B.Mask") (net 45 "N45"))
  (pad "3" smd rect (at 2.45 -1.65 90) (size 1.5 0.9) (layers "B.Cu" "B.Paste" "B.Mask") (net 2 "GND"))
  (pad "4" smd rect (at 2.45 1.65 90) (size 1.5 0.9) (layers "B.Cu" "B.Paste" "B.Mask") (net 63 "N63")))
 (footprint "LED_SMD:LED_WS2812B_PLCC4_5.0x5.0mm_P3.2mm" (layer "B.Cu") (at 155 145 -90)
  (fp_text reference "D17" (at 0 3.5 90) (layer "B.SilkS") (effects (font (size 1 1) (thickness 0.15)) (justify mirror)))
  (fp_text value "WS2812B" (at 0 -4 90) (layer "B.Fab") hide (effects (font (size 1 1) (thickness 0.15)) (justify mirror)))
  (pad "1" smd rect (at -2.45 1.65 270) (size 1.5 0.9) (layers "B.Cu" "B.Paste" "B.Mask") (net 1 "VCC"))
  (pad "2" smd rect (at -2.45 -1.65 270) (size 1.5 0.9) (layers "B.Cu" "B.Paste" "B.Mask") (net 52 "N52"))
  (pad "3" smd rect (at 2.45 -1.65 270) (size 1.5 0.9) (layers "B.Cu" "B.Paste" "B.Mask") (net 2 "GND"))
  (pad "4" smd rect (at 2.45 1.65 270) (size 1.5 0.9) (layers "B.Cu" "B.Paste" "B.Mask") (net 54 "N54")))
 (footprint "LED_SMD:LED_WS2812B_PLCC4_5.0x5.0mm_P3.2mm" (layer "B.Cu") (at 155 72.5 90)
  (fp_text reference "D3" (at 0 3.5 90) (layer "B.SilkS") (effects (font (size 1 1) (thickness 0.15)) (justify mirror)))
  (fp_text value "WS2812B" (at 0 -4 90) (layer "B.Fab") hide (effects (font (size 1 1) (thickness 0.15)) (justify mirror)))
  (pad "1" smd rect (at -2.45 1.65 90) (size 1.5 0.9) (layers "B.Cu" "B.Paste" "B.Mask") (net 1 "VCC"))
  (pad "2" smd rect (at -2.45 -1.65 90) (size 1.5 0.9) (layers "B.Cu" "B.Paste" "B.Mask") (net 63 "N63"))
  (pad "3" smd rect (at 2.45 -1.65 90) (size 1.5 0.9) (layers "B.Cu" "B.Paste" "B.Mask") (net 2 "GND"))
  (pad "4" smd rect (at 2.45 1.65 90) (size 1.5 0.9) (layers "B.Cu" "B.Paste" "B.Mask") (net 60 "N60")))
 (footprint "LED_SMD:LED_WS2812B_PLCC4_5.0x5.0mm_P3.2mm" (layer "B.Cu") (at 115 93.4 90)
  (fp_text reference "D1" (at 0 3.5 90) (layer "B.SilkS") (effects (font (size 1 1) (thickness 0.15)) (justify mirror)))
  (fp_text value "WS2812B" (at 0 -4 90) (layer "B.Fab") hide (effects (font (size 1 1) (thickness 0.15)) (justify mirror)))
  (pad "1" smd rect (at -2.45 1.65 90) (size 1.5 0.9) (layers "B.Cu" "B.Paste" "B.Mask") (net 1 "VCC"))
  (pad "2" smd rect (at -2.45 -1.65 90) (size 1.5 0.9) (layers "B.Cu" "B.Paste" "B.Mask") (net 49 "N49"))
  (pad "3" smd rect (at 2.45 -1.65 90) (size 1.5 0.9) (layers "B.Cu" "B.Paste" "B.Mask") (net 2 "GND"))
  (pad "4" smd rect (at 2.45 1.65 90) (size 1.5 0.9) (layers "B.Cu" "B.Paste" "B.Mask") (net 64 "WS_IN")))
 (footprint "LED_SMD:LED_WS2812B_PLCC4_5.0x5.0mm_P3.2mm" (layer "B.Cu") (at 115 135 90)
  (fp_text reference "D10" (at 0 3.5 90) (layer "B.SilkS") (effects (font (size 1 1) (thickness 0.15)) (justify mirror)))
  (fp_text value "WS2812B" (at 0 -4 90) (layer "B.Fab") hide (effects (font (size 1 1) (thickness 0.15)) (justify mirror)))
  (pad "1" smd rect (at -2.45 1.65 90) (size 1.5 0.9) (layers "B.Cu" "B.Paste" "B.Mask") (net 1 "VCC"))
  (pad "2" smd rect (at -2.45 -1.65 90) (size 1.5 0.9) (layers "B.Cu" "B.Paste" "B.Mask") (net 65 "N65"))
  (pad "3" smd rect (at 2.45 -1.65 90) (size 1.5 0.9) (layers "B.Cu" "B.Paste" "B.Mask") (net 2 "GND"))
  (pad "4" smd rect (at 2.45 1.65 90) (size 1.5 0.9) (layers "B.Cu" "B.Paste" "B.Mask") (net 59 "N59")))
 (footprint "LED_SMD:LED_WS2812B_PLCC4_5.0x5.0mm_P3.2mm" (layer "B.Cu") (at 125 65 180)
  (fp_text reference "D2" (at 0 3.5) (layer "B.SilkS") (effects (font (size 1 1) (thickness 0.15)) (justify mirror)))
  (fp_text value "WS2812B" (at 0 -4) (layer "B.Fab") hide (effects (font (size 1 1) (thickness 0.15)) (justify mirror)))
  (pad "1" smd rect (at -2.45 1.65 180) (size 1.5 0.9) (layers "B.Cu" "B.Paste" "B.Mask") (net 1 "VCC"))
  (pad "2" smd rect (at -2.45 -1.65 180) (size 1.5 0.9) (layers "B.Cu" "B.Paste" "B.Mask") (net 62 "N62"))
  (pad "3" smd rect (at 2.45 -1.65 180) (size 1.5 0.9) (layers "B.Cu" "B.Paste" "B.Mask") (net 2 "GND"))
  (pad "4" smd rect (at 2.45 1.65 180) (size 1.5 0.9) (layers "B.Cu" "B.Paste" "B.Mask") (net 53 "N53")))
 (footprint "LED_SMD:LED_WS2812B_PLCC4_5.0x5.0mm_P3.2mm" (layer "B.Cu") (at 115 145 90)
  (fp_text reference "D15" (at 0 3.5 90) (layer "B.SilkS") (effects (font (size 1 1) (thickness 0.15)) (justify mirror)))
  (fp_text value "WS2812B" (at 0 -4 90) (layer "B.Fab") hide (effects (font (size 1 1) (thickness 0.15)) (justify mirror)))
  (pad "1" smd rect (at -2.45 1.65 90) (size 1.5 0.9) (layers "B.Cu" "B.Paste" "B.Mask") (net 1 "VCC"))
  (pad "2" smd rect (at -2.45 -1.65 90) (size 1.5 0.9) (layers "B.Cu" "B.Paste" "B.Mask") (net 57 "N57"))
  (pad "3" smd rect (at 2.45 -1.65 90) (size 1.5 0.9) (layers "B.Cu" "B.Paste" "B.Mask") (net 2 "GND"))
  (pad "4" smd rect (at 2.45 1.65 90) (size 1.5 0.9) (layers "B.Cu" "B.Paste" "B.Mask") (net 65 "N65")))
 (gr_line (start 160 120) (end 160 150) (layer "Edge.Cuts") (width 0.1))
 (gr_line (start 120 125) (end 125 120) (layer "Edge.Cuts") (width 0.1))
 (gr_line (start 150 60) (end 120 60) (layer "Edge.Cuts") (width 0.1))
 (gr_line (start 120 145) (end 120 125) (layer "Edge.Cuts") (width 0.1))
 (gr_line (start 150 95) (end 150 75) (layer "Edge.Cuts") (width 0.1))
 (gr_line (start 150 145) (end 145 150) (layer "Edge.Cuts") (width 0.1))
 (gr_line (start 110 150) (end 120 160) (layer "Edge.Cuts") (width 0.1))
 (gr_line (start 120 95) (end 125 100) (layer "Edge.Cuts") (width 0.1))
 (gr_line (start 120 75) (end 120 95) (layer "Edge.Cuts") (width 0.1))
 (gr_line (start 120 160) (end 150 160) (layer "Edge.Cuts") (width 0.1))
 (gr_line (start 120 110) (end 110 120) (layer "Edge.Cuts") (width 0.1))
 (gr_line (start 160 120) (end 150 110) (layer "Edge.Cuts") (width 0.1))
 (gr_line (start 145 100) (end 150 95) (layer "Edge.Cuts") (width 0.1))
 (gr_line (start 110 70) (end 110 100) (layer "Edge.Cuts") (width 0.1))
 (gr_line (start 125 150) (end 120 145) (layer "Edge.Cuts") (width 0.1))
 (gr_line (start 150 160) (end 160 150) (layer "Edge.Cuts") (width 0.1))
 (gr_line (start 145 70) (end 125 70) (layer "Edge.Cuts") (width 0.1))
 (gr_line (start 150 125) (end 150 145) (layer "Edge.Cuts") (width 0.1))
 (gr_line (start 160 100) (end 150 110) (layer "Edge.Cuts") (width 0.1))
 (gr_line (start 150 75) (end 145 70) (layer "Edge.Cuts") (width 0.1))
 (gr_line (start 125 120) (end 145 120) (layer "Edge.Cuts") (width 0.1))
 (gr_line (start 125 70) (end 120 75) (layer "Edge.Cuts") (width 0.1))
 (gr_line (start 145 150) (end 125 150) (layer "Edge.Cuts") (width 0.1))
 (gr_line (start 125 100) (end 145 100) (layer "Edge.Cuts") (width 0.1))
 (gr_line (start 160 70) (end 150 60) (layer "Edge.Cuts") (width 0.1))
 (gr_line (start 110 100) (end 120 110) (layer "Edge.Cuts") (width 0.1))
 (gr_line (start 160 100) (end 160 70) (layer "Edge.Cuts") (width 0.1))
 (gr_line (start 145 120) (end 150 125) (layer "Edge.Cuts") (width 0.1))
 (gr_line (start 110 120) (end 110 150) (layer "Edge.Cuts") (width 0.1))
 (gr_line (start 120 60) (end 110 70) (layer "Edge.Cuts") (width 0.1))
 (segment (start 140.425 113.03) (end 137.605 113.03) (width 0.25) (layer "F.Cu") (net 1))
 (segment (start 137.2 110.875) (end 137.2 112.475) (width 0.25) (layer "F.Cu") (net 1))
 (segment (start 137.2 112.475) (end 137.125 112.55) (width 0.25) (layer "F.Cu") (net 1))
 (segment (start 135.525 110.875) (end 137.2 110.875) (width 0.25) (layer "F.Cu") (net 1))
 (segment (start 137.605 113.03) (end 137.125 112.55) (width 0.25) (layer "F.Cu") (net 1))
 (segment (start 137.205 109.22) (end 137.2 109.225) (width 0.25) (layer "F.Cu") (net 6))
 (segment (start 140.425 109.22) (end 137.205 109.22) (width 0.25) (layer "F.Cu") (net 6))
 (segment (start 136.45 110.15) (end 135.525 109.225) (width 0.25) (layer "F.Cu") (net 7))
 (segment (start 140.425 110.49) (end 140.085 110.15) (width 0.25) (layer "F.Cu") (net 7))
 (segment (start 140.085 110.15) (end 136.45 110.15) (width 0.25) (layer "F.Cu") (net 7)))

